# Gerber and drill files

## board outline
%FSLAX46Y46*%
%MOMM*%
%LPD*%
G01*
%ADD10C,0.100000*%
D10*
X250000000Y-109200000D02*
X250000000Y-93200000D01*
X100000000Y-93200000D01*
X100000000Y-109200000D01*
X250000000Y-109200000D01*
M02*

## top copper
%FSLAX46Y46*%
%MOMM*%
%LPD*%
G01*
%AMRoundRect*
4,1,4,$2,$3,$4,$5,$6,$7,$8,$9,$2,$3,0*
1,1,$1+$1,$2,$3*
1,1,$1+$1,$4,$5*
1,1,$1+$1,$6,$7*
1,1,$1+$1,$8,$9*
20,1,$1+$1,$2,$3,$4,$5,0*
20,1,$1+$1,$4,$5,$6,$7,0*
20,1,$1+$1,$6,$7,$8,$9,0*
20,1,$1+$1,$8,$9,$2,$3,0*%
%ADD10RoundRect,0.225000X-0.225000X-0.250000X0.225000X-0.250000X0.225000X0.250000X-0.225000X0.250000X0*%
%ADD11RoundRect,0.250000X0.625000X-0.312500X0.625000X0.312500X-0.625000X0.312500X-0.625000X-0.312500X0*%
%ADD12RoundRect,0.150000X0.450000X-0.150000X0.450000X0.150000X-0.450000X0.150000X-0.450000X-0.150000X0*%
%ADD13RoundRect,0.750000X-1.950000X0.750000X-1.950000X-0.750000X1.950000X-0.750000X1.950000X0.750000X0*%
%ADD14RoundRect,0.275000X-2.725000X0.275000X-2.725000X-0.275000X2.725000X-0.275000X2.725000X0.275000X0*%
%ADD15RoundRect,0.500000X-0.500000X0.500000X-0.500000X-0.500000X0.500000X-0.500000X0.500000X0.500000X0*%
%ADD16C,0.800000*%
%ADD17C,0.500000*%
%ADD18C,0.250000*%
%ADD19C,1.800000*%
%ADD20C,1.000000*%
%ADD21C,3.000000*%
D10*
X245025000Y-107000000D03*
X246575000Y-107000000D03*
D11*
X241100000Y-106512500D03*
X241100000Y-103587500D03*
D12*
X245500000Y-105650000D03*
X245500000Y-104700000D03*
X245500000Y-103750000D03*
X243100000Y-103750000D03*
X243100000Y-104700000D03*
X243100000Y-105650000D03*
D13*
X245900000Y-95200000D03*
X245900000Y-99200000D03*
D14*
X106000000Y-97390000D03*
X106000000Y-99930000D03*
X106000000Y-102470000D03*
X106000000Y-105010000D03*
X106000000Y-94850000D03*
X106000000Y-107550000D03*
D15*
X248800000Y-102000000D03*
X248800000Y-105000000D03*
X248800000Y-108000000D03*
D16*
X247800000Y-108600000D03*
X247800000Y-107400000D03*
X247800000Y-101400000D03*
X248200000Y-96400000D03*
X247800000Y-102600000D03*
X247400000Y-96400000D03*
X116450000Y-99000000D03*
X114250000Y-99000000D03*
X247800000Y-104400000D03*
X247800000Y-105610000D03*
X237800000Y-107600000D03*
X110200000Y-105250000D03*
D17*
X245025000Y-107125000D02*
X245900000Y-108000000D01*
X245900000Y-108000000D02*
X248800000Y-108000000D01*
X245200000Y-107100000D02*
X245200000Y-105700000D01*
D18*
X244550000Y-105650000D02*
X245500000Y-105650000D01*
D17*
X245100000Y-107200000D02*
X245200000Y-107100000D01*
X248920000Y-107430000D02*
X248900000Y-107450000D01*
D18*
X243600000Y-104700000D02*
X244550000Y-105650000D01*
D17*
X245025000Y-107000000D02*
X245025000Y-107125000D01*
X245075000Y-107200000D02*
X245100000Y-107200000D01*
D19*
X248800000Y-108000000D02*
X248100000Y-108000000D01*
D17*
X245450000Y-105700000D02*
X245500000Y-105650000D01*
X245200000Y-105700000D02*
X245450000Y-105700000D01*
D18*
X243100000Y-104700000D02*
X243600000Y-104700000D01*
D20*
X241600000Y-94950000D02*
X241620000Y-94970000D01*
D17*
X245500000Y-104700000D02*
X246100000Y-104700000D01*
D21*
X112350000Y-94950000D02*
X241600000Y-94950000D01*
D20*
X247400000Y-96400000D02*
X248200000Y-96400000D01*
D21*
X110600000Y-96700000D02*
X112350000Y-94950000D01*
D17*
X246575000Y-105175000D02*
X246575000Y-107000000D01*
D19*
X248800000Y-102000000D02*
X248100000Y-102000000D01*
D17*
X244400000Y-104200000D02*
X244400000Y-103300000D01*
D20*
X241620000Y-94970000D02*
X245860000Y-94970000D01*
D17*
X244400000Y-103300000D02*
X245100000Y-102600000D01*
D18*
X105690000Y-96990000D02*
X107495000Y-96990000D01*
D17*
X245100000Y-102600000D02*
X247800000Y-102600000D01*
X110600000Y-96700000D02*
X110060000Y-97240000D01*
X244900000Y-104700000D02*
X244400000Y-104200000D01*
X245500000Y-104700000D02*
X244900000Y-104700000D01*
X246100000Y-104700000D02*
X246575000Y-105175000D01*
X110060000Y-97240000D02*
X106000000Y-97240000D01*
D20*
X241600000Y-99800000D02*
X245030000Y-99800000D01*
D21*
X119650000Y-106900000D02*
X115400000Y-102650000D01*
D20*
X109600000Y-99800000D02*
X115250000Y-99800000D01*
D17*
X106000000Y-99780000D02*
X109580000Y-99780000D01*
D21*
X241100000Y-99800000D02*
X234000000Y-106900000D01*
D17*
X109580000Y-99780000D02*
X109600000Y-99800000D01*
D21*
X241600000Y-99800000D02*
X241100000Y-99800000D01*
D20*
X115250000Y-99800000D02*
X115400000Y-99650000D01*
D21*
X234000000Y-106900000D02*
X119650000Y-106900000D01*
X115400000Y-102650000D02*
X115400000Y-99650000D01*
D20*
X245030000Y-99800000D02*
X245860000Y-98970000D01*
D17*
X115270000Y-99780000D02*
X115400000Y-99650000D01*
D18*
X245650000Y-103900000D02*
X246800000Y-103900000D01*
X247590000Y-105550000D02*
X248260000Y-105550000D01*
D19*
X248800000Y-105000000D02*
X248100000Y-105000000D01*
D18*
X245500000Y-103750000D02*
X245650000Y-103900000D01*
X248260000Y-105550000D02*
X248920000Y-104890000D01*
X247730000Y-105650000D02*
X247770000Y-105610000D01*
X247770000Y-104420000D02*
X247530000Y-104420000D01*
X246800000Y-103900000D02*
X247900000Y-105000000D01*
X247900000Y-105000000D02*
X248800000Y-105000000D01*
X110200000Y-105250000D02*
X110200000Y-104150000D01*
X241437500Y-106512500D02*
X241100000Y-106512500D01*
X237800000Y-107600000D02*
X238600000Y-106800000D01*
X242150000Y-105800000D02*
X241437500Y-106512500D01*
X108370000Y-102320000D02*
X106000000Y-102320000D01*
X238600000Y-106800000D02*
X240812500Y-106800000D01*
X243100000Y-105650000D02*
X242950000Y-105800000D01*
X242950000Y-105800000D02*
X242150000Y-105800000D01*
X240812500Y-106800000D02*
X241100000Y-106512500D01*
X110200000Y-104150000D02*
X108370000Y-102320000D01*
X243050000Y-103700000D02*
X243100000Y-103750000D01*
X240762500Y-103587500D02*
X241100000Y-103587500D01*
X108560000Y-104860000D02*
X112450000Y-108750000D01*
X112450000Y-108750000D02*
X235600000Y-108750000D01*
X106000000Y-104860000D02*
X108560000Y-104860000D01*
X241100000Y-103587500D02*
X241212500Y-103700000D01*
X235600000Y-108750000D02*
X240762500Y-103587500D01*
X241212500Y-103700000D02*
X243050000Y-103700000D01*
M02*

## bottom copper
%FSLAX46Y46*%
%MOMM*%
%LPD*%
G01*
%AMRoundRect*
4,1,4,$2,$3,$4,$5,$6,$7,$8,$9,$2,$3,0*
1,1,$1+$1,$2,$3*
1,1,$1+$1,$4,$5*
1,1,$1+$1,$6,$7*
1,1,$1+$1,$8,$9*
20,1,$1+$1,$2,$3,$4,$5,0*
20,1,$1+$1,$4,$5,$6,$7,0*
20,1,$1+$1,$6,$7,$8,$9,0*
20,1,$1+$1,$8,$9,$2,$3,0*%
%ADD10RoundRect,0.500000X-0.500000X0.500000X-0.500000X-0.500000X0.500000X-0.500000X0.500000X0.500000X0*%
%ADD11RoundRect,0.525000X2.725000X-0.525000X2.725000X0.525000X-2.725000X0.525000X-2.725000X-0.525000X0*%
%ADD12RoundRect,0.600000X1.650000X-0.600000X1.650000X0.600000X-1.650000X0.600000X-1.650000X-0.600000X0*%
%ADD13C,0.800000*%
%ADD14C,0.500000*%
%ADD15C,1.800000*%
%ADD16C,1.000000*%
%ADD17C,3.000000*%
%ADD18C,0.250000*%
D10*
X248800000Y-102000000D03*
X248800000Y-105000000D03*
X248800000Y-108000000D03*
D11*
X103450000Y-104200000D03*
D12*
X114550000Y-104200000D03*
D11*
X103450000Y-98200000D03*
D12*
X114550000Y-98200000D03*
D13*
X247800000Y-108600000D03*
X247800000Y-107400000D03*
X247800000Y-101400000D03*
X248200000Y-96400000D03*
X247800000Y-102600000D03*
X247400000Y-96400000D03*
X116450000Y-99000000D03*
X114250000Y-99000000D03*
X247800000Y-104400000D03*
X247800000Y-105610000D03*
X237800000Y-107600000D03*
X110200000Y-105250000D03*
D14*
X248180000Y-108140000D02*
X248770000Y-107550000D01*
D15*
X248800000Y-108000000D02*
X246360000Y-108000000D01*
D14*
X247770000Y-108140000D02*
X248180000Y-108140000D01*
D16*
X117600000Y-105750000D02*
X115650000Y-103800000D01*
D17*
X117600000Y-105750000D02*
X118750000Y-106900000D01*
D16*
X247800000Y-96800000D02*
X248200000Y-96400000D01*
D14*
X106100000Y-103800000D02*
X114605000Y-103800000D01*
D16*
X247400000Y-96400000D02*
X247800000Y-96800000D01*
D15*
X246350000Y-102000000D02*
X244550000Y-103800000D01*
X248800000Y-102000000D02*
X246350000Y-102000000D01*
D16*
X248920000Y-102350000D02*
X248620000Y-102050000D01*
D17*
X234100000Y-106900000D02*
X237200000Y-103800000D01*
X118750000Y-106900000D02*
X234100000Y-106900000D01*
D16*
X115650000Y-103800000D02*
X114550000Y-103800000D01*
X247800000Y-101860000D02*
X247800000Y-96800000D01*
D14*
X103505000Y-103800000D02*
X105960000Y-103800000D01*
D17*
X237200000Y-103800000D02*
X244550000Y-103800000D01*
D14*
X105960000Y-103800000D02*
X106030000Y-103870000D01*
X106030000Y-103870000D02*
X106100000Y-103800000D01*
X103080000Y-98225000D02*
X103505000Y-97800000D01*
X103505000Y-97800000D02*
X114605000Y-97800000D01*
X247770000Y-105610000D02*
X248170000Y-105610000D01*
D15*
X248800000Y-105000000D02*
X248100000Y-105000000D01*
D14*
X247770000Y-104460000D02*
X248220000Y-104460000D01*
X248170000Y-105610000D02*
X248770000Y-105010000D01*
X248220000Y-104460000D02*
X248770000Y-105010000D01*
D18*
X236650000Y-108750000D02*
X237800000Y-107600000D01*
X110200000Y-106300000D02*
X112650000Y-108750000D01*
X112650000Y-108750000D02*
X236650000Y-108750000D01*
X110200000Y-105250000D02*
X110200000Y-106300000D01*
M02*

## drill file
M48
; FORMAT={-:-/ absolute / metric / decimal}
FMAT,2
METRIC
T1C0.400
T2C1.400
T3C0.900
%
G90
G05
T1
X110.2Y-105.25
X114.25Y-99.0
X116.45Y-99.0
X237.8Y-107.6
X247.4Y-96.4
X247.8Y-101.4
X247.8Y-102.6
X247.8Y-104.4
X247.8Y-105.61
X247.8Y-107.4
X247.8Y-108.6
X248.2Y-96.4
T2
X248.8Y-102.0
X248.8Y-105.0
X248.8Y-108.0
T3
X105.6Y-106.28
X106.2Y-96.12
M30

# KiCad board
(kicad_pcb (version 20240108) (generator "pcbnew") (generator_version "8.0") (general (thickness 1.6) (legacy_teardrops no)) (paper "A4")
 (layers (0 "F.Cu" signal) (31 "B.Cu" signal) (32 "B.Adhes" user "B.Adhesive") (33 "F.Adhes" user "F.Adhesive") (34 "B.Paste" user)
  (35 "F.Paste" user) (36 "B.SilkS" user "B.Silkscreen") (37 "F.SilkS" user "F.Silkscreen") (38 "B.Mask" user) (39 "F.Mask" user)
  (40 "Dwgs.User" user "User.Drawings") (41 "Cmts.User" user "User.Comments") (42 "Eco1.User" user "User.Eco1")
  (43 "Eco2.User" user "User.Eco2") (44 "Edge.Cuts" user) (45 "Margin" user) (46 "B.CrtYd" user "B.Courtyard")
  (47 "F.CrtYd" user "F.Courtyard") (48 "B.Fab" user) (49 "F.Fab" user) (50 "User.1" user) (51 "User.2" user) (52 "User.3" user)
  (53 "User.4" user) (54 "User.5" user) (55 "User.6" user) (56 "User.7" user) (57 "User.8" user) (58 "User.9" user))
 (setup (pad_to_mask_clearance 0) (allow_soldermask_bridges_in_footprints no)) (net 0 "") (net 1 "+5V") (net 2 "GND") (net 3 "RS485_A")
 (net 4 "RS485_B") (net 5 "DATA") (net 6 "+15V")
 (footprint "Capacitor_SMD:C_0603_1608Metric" (layer "F.Cu") (at 245.8 107)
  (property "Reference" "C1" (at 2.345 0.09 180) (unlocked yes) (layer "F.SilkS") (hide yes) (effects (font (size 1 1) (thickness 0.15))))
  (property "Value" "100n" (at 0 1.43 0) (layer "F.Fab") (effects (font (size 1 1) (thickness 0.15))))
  (pad "1" smd roundrect (at -0.775 0) (size 0.9 0.95) (layers "F.Cu" "F.Paste" "F.Mask") (roundrect_rratio 0.25) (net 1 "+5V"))
  (pad "2" smd roundrect (at 0.775 0) (size 0.9 0.95) (layers "F.Cu" "F.Paste" "F.Mask") (roundrect_rratio 0.25) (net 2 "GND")))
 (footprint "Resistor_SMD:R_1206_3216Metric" (layer "F.Cu") (at 241.1 105.05 90)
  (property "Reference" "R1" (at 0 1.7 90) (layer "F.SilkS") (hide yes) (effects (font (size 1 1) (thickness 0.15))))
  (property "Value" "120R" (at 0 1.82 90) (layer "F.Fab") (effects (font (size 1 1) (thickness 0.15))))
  (pad "1" smd roundrect (at -1.4625 0 90) (size 1.125 1.75) (layers "F.Cu" "F.Paste" "F.Mask") (roundrect_rratio 0.222222)
   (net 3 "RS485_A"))
  (pad "2" smd roundrect (at 1.4625 0 90) (size 1.125 1.75) (layers "F.Cu" "F.Paste" "F.Mask") (roundrect_rratio 0.222222) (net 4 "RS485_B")))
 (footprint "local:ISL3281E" (layer "F.Cu") (at 244.3 104.7 90)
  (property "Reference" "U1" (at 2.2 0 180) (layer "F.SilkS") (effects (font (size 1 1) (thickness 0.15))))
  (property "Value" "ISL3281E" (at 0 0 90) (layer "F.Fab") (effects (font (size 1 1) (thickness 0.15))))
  (pad "1" smd roundrect (at -0.95 1.2 90) (size 0.6 1.2) (layers "F.Cu" "F.Paste" "F.Mask") (roundrect_rratio 0.25) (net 1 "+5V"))
  (pad "2" smd roundrect (at 0 1.2 90) (size 0.6 1.2) (layers "F.Cu" "F.Paste" "F.Mask") (roundrect_rratio 0.25) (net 2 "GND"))
  (pad "3" smd roundrect (at 0.95 1.2 90) (size 0.6 1.2) (layers "F.Cu" "F.Paste" "F.Mask") (roundrect_rratio 0.25) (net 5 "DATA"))
  (pad "4" smd roundrect (at 0.95 -1.2 90) (size 0.6 1.2) (layers "F.Cu" "F.Paste" "F.Mask") (roundrect_rratio 0.25) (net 4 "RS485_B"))
  (pad "5" smd roundrect (at 0 -1.2 90) (size 0.6 1.2) (layers "F.Cu" "F.Paste" "F.Mask") (roundrect_rratio 0.25) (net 1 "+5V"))
  (pad "6" smd roundrect (at -0.95 -1.2 90) (size 0.6 1.2) (layers "F.Cu" "F.Paste" "F.Mask") (roundrect_rratio 0.25) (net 3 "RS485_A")))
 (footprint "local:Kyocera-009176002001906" (layer "F.Cu") (at 245.9 97.2 -90)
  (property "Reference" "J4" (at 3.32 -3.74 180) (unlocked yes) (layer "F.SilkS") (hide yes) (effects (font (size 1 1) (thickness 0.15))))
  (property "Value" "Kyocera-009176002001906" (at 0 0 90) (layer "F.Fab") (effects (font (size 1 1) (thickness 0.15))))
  (pad "1" smd roundrect (at -2 0 270) (size 3 5.4) (layers "F.Cu" "F.Paste" "F.Mask") (roundrect_rratio 0.25) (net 2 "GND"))
  (pad "2" smd roundrect (at 2 0 270) (size 3 5.4) (layers "F.Cu" "F.Paste" "F.Mask") (roundrect_rratio 0.25) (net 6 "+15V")))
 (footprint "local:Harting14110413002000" (layer "F.Cu") (at 106 101.2 -90)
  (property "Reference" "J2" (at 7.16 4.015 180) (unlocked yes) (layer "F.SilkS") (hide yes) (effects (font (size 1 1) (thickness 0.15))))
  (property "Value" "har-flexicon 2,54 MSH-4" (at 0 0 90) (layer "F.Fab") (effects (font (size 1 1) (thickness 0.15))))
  (pad "" np_thru_hole circle (at -5.08 -0.2 270) (size 0.9 0.9) (drill 0.9) (layers "*.Cu" "*.Mask"))
  (pad "" np_thru_hole circle (at 5.08 0.4 270) (size 0.9 0.9) (drill 0.9) (layers "*.Cu" "*.Mask"))
  (pad "1" smd roundrect (at -3.81 0 270) (size 1.1 6) (layers "F.Cu" "F.Paste" "F.Mask") (roundrect_rratio 0.25) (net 2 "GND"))
  (pad "2" smd roundrect (at -1.27 0 270) (size 1.1 6) (layers "F.Cu" "F.Paste" "F.Mask") (roundrect_rratio 0.25) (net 6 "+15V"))
  (pad "3" smd roundrect (at 1.27 0 270) (size 1.1 6) (layers "F.Cu" "F.Paste" "F.Mask") (roundrect_rratio 0.25) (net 3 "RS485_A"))
  (pad "4" smd roundrect (at 3.81 0 270) (size 1.1 6) (layers "F.Cu" "F.Paste" "F.Mask") (roundrect_rratio 0.25) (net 4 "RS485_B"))
  (pad "MP1" smd roundrect (at -6.35 0 270) (size 1.1 6) (layers "F.Cu" "F.Paste" "F.Mask") (roundrect_rratio 0.25))
  (pad "MP2" smd roundrect (at 6.35 0 270) (size 1.1 6) (layers "F.Cu" "F.Paste" "F.Mask") (roundrect_rratio 0.25)))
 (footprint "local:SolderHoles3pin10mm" (layer "F.Cu") (at 248.8 105 -90)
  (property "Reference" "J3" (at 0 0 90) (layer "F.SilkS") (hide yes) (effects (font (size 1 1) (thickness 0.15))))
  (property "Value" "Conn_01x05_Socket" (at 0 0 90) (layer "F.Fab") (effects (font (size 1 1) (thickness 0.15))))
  (pad "1" thru_hole roundrect (at -3 0 270) (size 2 2) (drill 1.4) (layers "*.Cu" "*.Mask") (remove_unused_layers yes)
   (keep_end_layers yes) (zone_layer_connections) (roundrect_rratio 0.25) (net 2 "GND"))
  (pad "2" thru_hole roundrect (at 0 0 270) (size 2 2) (drill 1.4) (layers "*.Cu" "*.Mask") (remove_unused_layers yes) (keep_end_layers yes)
   (zone_layer_connections) (roundrect_rratio 0.25) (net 5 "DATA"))
  (pad "3" thru_hole roundrect (at 3 0 270) (size 2 2) (drill 1.4) (layers "*.Cu" "*.Mask") (remove_unused_layers yes) (keep_end_layers yes)
   (zone_layer_connections) (roundrect_rratio 0.25) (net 1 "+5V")))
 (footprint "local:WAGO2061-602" (layer "B.Cu") (at 108.2 101.2 90)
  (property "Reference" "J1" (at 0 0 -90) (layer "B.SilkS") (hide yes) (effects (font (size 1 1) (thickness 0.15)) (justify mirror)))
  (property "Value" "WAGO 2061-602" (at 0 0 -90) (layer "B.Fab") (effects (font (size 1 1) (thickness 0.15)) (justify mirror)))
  (pad "1" smd roundrect (at -3 -4.75 90) (size 2.1 6.5) (layers "B.Cu" "B.Paste" "B.Mask") (roundrect_rratio 0.25) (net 2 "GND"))
  (pad "1" smd roundrect (at -3 6.35 90) (size 2.4 4.5) (layers "B.Cu" "B.Paste" "B.Mask") (roundrect_rratio 0.25) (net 2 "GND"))
  (pad "2" smd roundrect (at 3 -4.75 90) (size 2.1 6.5) (layers "B.Cu" "B.Paste" "B.Mask") (roundrect_rratio 0.25) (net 6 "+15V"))
  (pad "2" smd roundrect (at 3 6.35 90) (size 2.4 4.5) (layers "B.Cu" "B.Paste" "B.Mask") (roundrect_rratio 0.25) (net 6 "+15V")))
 (gr_poly (pts (xy 250 109.2) (xy 250 93.2) (xy 100 93.2) (xy 100 109.2)) (stroke (width 0.1) (type solid)) (fill none) (layer "Edge.Cuts"))
 (segment (start 245.025 107.125) (end 245.9 108) (width 0.5) (layer "F.Cu") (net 1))
 (segment (start 245.9 108) (end 248.8 108) (width 0.5) (layer "F.Cu") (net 1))
 (segment (start 245.2 107.1) (end 245.2 105.7) (width 0.5) (layer "F.Cu") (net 1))
 (segment (start 244.55 105.65) (end 245.5 105.65) (width 0.25) (layer "F.Cu") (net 1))
 (segment (start 245.1 107.2) (end 245.2 107.1) (width 0.5) (layer "F.Cu") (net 1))
 (segment (start 248.92 107.43) (end 248.9 107.45) (width 0.5) (layer "F.Cu") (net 1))
 (segment (start 243.6 104.7) (end 244.55 105.65) (width 0.25) (layer "F.Cu") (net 1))
 (segment (start 245.025 107) (end 245.025 107.125) (width 0.5) (layer "F.Cu") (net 1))
 (segment (start 245.075 107.2) (end 245.1 107.2) (width 0.5) (layer "F.Cu") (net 1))
 (segment (start 248.8 108) (end 248.1 108) (width 1.8) (layer "F.Cu") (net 1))
 (segment (start 245.45 105.7) (end 245.5 105.65) (width 0.5) (layer "F.Cu") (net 1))
 (segment (start 245.2 105.7) (end 245.45 105.7) (width 0.5) (layer "F.Cu") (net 1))
 (segment (start 243.1 104.7) (end 243.6 104.7) (width 0.25) (layer "F.Cu") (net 1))
 (via (at 247.8 108.6) (size 0.8) (drill 0.4) (layers "F.Cu" "B.Cu") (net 1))
 (via (at 247.8 107.4) (size 0.8) (drill 0.4) (layers "F.Cu" "B.Cu") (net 1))
 (segment (start 248.18 108.14) (end 248.77 107.55) (width 0.5) (layer "B.Cu") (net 1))
 (segment (start 248.8 108) (end 246.36 108) (width 1.8) (layer "B.Cu") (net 1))
 (segment (start 247.77 108.14) (end 248.18 108.14) (width 0.5) (layer "B.Cu") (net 1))
 (segment (start 241.6 94.95) (end 241.62 94.97) (width 1) (layer "F.Cu") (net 2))
 (segment (start 245.5 104.7) (end 246.1 104.7) (width 0.5) (layer "F.Cu") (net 2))
 (segment (start 112.35 94.95) (end 241.6 94.95) (width 3) (layer "F.Cu") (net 2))
 (segment (start 247.4 96.4) (end 248.2 96.4) (width 1) (layer "F.Cu") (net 2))
 (segment (start 110.6 96.7) (end 112.35 94.95) (width 3) (layer "F.Cu") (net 2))
 (segment (start 246.575 105.175) (end 246.575 107) (width 0.5) (layer "F.Cu") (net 2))
 (segment (start 248.8 102) (end 248.1 102) (width 1.8) (layer "F.Cu") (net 2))
 (segment (start 244.4 104.2) (end 244.4 103.3) (width 0.5) (layer "F.Cu") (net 2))
 (segment (start 241.62 94.97) (end 245.86 94.97) (width 1) (layer "F.Cu") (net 2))
 (segment (start 244.4 103.3) (end 245.1 102.6) (width 0.5) (layer "F.Cu") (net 2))
 (segment (start 105.69 96.99) (end 107.495 96.99) (width 0.25) (layer "F.Cu") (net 2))
 (segment (start 245.1 102.6) (end 247.8 102.6) (width 0.5) (layer "F.Cu") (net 2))
 (segment (start 110.6 96.7) (end 110.06 97.24) (width 0.5) (layer "F.Cu") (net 2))
 (segment (start 244.9 104.7) (end 244.4 104.2) (width 0.5) (layer "F.Cu") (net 2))
 (segment (start 245.5 104.7) (end 244.9 104.7) (width 0.5) (layer "F.Cu") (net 2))
 (segment (start 246.1 104.7) (end 246.575 105.175) (width 0.5) (layer "F.Cu") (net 2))
 (segment (start 110.06 97.24) (end 106 97.24) (width 0.5) (layer "F.Cu") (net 2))
 (via (at 247.8 101.4) (size 0.8) (drill 0.4) (layers "F.Cu" "B.Cu") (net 2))
 (via (at 248.2 96.4) (size 0.8) (drill 0.4) (layers "F.Cu" "B.Cu") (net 2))
 (via (at 247.8 102.6) (size 0.8) (drill 0.4) (layers "F.Cu" "B.Cu") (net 2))
 (via (at 247.4 96.4) (size 0.8) (drill 0.4) (layers "F.Cu" "B.Cu") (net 2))
 (segment (start 117.6 105.75) (end 115.65 103.8) (width 1) (layer "B.Cu") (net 2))
 (segment (start 117.6 105.75) (end 118.75 106.9) (width 3) (layer "B.Cu") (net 2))
 (segment (start 247.8 96.8) (end 248.2 96.4) (width 1) (layer "B.Cu") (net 2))
 (segment (start 106.1 103.8) (end 114.605 103.8) (width 0.5) (layer "B.Cu") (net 2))
 (segment (start 247.4 96.4) (end 247.8 96.8) (width 1) (layer "B.Cu") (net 2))
 (segment (start 246.35 102) (end 244.55 103.8) (width 1.8) (layer "B.Cu") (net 2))
 (segment (start 248.8 102) (end 246.35 102) (width 1.8) (layer "B.Cu") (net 2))
 (segment (start 248.92 102.35) (end 248.62 102.05) (width 1) (layer "B.Cu") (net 2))
 (segment (start 234.1 106.9) (end 237.2 103.8) (width 3) (layer "B.Cu") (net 2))
 (segment (start 118.75 106.9) (end 234.1 106.9) (width 3) (layer "B.Cu") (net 2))
 (segment (start 115.65 103.8) (end 114.55 103.8) (width 1) (layer "B.Cu") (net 2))
 (segment (start 247.8 101.86) (end 247.8 96.8) (width 1) (layer "B.Cu") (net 2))
 (segment (start 103.505 103.8) (end 105.96 103.8) (width 0.5) (layer "B.Cu") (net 2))
 (segment (start 237.2 103.8) (end 244.55 103.8) (width 3) (layer "B.Cu") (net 2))
 (segment (start 105.96 103.8) (end 106.03 103.87) (width 0.5) (layer "B.Cu") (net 2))
 (segment (start 106.03 103.87) (end 106.1 103.8) (width 0.5) (layer "B.Cu") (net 2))
 (segment (start 241.6 99.8) (end 245.03 99.8) (width 1) (layer "F.Cu") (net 6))
 (segment (start 119.65 106.9) (end 115.4 102.65) (width 3) (layer "F.Cu") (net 6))
 (segment (start 109.6 99.8) (end 115.25 99.8) (width 1) (layer "F.Cu") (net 6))
 (segment (start 106 99.78) (end 109.58 99.78) (width 0.5) (layer "F.Cu") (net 6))
 (segment (start 241.1 99.8) (end 234 106.9) (width 3) (layer "F.Cu") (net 6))
 (segment (start 109.58 99.78) (end 109.6 99.8) (width 0.5) (layer "F.Cu") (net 6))
 (segment (start 241.6 99.8) (end 241.1 99.8) (width 3) (layer "F.Cu") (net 6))
 (segment (start 115.25 99.8) (end 115.4 99.65) (width 1) (layer "F.Cu") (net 6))
 (segment (start 234 106.9) (end 119.65 106.9) (width 3) (layer "F.Cu") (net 6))
 (segment (start 115.4 102.65) (end 115.4 99.65) (width 3) (layer "F.Cu") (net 6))
 (segment (start 245.03 99.8) (end 245.86 98.97) (width 1) (layer "F.Cu") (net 6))
 (segment (start 115.27 99.78) (end 115.4 99.65) (width 0.5) (layer "F.Cu") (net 6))
 (via (at 116.45 99) (size 0.8) (drill 0.4) (layers "F.Cu" "B.Cu") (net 6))
 (via (at 114.25 99) (size 0.8) (drill 0.4) (layers "F.Cu" "B.Cu") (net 6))
 (segment (start 103.08 98.225) (end 103.505 97.8) (width 0.5) (layer "B.Cu") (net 6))
 (segment (start 103.505 97.8) (end 114.605 97.8) (width 0.5) (layer "B.Cu") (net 6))
 (segment (start 245.65 103.9) (end 246.8 103.9) (width 0.25) (layer "F.Cu") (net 5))
 (segment (start 247.59 105.55) (end 248.26 105.55) (width 0.25) (layer "F.Cu") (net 5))
 (segment (start 248.8 105) (end 248.1 105) (width 1.8) (layer "F.Cu") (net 5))
 (segment (start 245.5 103.75) (end 245.65 103.9) (width 0.25) (layer "F.Cu") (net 5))
 (segment (start 248.26 105.55) (end 248.92 104.89) (width 0.25) (layer "F.Cu") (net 5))
 (segment (start 247.73 105.65) (end 247.77 105.61) (width 0.25) (layer "F.Cu") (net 5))
 (segment (start 247.77 104.42) (end 247.53 104.42) (width 0.25) (layer "F.Cu") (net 5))
 (segment (start 246.8 103.9) (end 247.9 105) (width 0.25) (layer "F.Cu") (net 5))
 (segment (start 247.9 105) (end 248.8 105) (width 0.25) (layer "F.Cu") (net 5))
 (via (at 247.8 104.4) (size 0.8) (drill 0.4) (layers "F.Cu" "B.Cu") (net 5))
 (via (at 247.8 105.61) (size 0.8) (drill 0.4) (layers "F.Cu" "B.Cu") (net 5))
 (segment (start 247.77 105.61) (end 248.17 105.61) (width 0.5) (layer "B.Cu") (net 5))
 (segment (start 248.8 105) (end 248.1 105) (width 1.8) (layer "B.Cu") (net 5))
 (segment (start 247.77 104.46) (end 248.22 104.46) (width 0.5) (layer "B.Cu") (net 5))
 (segment (start 248.17 105.61) (end 248.77 105.01) (width 0.5) (layer "B.Cu") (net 5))
 (segment (start 248.22 104.46) (end 248.77 105.01) (width 0.5) (layer "B.Cu") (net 5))
 (segment (start 110.2 105.25) (end 110.2 104.15) (width 0.25) (layer "F.Cu") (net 3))
 (segment (start 241.4375 106.5125) (end 241.1 106.5125) (width 0.25) (layer "F.Cu") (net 3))
 (segment (start 237.8 107.6) (end 238.6 106.8) (width 0.25) (layer "F.Cu") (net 3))
 (segment (start 242.15 105.8) (end 241.4375 106.5125) (width 0.25) (layer "F.Cu") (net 3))
 (segment (start 108.37 102.32) (end 106 102.32) (width 0.25) (layer "F.Cu") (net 3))
 (segment (start 238.6 106.8) (end 240.8125 106.8) (width 0.25) (layer "F.Cu") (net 3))
 (segment (start 243.1 105.65) (end 242.95 105.8) (width 0.25) (layer "F.Cu") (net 3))
 (segment (start 242.95 105.8) (end 242.15 105.8) (width 0.25) (layer "F.Cu") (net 3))
 (segment (start 240.8125 106.8) (end 241.1 106.5125) (width 0.25) (layer "F.Cu") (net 3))
 (segment (start 110.2 104.15) (end 108.37 102.32) (width 0.25) (layer "F.Cu") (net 3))
 (via (at 237.8 107.6) (size 0.8) (drill 0.4) (layers "F.Cu" "B.Cu") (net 3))
 (via (at 110.2 105.25) (size 0.8) (drill 0.4) (layers "F.Cu" "B.Cu") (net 3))
 (segment (start 236.65 108.75) (end 237.8 107.6) (width 0.25) (layer "B.Cu") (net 3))
 (segment (start 110.2 106.3) (end 112.65 108.75) (width 0.25) (layer "B.Cu") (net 3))
 (segment (start 112.65 108.75) (end 236.65 108.75) (width 0.25) (layer "B.Cu") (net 3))
 (segment (start 110.2 105.25) (end 110.2 106.3) (width 0.25) (layer "B.Cu") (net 3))
 (segment (start 243.05 103.7) (end 243.1 103.75) (width 0.25) (layer "F.Cu") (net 4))
 (segment (start 240.7625 103.5875) (end 241.1 103.5875) (width 0.25) (layer "F.Cu") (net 4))
 (segment (start 108.56 104.86) (end 112.45 108.75) (width 0.25) (layer "F.Cu") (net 4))
 (segment (start 112.45 108.75) (end 235.6 108.75) (width 0.25) (layer "F.Cu") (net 4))
 (segment (start 106 104.86) (end 108.56 104.86) (width 0.25) (layer "F.Cu") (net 4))
 (segment (start 241.1 103.5875) (end 241.2125 103.7) (width 0.25) (layer "F.Cu") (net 4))
 (segment (start 235.6 108.75) (end 240.7625 103.5875) (width 0.25) (layer "F.Cu") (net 4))
 (segment (start 241.2125 103.7) (end 243.05 103.7) (width 0.25) (layer "F.Cu") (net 4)))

